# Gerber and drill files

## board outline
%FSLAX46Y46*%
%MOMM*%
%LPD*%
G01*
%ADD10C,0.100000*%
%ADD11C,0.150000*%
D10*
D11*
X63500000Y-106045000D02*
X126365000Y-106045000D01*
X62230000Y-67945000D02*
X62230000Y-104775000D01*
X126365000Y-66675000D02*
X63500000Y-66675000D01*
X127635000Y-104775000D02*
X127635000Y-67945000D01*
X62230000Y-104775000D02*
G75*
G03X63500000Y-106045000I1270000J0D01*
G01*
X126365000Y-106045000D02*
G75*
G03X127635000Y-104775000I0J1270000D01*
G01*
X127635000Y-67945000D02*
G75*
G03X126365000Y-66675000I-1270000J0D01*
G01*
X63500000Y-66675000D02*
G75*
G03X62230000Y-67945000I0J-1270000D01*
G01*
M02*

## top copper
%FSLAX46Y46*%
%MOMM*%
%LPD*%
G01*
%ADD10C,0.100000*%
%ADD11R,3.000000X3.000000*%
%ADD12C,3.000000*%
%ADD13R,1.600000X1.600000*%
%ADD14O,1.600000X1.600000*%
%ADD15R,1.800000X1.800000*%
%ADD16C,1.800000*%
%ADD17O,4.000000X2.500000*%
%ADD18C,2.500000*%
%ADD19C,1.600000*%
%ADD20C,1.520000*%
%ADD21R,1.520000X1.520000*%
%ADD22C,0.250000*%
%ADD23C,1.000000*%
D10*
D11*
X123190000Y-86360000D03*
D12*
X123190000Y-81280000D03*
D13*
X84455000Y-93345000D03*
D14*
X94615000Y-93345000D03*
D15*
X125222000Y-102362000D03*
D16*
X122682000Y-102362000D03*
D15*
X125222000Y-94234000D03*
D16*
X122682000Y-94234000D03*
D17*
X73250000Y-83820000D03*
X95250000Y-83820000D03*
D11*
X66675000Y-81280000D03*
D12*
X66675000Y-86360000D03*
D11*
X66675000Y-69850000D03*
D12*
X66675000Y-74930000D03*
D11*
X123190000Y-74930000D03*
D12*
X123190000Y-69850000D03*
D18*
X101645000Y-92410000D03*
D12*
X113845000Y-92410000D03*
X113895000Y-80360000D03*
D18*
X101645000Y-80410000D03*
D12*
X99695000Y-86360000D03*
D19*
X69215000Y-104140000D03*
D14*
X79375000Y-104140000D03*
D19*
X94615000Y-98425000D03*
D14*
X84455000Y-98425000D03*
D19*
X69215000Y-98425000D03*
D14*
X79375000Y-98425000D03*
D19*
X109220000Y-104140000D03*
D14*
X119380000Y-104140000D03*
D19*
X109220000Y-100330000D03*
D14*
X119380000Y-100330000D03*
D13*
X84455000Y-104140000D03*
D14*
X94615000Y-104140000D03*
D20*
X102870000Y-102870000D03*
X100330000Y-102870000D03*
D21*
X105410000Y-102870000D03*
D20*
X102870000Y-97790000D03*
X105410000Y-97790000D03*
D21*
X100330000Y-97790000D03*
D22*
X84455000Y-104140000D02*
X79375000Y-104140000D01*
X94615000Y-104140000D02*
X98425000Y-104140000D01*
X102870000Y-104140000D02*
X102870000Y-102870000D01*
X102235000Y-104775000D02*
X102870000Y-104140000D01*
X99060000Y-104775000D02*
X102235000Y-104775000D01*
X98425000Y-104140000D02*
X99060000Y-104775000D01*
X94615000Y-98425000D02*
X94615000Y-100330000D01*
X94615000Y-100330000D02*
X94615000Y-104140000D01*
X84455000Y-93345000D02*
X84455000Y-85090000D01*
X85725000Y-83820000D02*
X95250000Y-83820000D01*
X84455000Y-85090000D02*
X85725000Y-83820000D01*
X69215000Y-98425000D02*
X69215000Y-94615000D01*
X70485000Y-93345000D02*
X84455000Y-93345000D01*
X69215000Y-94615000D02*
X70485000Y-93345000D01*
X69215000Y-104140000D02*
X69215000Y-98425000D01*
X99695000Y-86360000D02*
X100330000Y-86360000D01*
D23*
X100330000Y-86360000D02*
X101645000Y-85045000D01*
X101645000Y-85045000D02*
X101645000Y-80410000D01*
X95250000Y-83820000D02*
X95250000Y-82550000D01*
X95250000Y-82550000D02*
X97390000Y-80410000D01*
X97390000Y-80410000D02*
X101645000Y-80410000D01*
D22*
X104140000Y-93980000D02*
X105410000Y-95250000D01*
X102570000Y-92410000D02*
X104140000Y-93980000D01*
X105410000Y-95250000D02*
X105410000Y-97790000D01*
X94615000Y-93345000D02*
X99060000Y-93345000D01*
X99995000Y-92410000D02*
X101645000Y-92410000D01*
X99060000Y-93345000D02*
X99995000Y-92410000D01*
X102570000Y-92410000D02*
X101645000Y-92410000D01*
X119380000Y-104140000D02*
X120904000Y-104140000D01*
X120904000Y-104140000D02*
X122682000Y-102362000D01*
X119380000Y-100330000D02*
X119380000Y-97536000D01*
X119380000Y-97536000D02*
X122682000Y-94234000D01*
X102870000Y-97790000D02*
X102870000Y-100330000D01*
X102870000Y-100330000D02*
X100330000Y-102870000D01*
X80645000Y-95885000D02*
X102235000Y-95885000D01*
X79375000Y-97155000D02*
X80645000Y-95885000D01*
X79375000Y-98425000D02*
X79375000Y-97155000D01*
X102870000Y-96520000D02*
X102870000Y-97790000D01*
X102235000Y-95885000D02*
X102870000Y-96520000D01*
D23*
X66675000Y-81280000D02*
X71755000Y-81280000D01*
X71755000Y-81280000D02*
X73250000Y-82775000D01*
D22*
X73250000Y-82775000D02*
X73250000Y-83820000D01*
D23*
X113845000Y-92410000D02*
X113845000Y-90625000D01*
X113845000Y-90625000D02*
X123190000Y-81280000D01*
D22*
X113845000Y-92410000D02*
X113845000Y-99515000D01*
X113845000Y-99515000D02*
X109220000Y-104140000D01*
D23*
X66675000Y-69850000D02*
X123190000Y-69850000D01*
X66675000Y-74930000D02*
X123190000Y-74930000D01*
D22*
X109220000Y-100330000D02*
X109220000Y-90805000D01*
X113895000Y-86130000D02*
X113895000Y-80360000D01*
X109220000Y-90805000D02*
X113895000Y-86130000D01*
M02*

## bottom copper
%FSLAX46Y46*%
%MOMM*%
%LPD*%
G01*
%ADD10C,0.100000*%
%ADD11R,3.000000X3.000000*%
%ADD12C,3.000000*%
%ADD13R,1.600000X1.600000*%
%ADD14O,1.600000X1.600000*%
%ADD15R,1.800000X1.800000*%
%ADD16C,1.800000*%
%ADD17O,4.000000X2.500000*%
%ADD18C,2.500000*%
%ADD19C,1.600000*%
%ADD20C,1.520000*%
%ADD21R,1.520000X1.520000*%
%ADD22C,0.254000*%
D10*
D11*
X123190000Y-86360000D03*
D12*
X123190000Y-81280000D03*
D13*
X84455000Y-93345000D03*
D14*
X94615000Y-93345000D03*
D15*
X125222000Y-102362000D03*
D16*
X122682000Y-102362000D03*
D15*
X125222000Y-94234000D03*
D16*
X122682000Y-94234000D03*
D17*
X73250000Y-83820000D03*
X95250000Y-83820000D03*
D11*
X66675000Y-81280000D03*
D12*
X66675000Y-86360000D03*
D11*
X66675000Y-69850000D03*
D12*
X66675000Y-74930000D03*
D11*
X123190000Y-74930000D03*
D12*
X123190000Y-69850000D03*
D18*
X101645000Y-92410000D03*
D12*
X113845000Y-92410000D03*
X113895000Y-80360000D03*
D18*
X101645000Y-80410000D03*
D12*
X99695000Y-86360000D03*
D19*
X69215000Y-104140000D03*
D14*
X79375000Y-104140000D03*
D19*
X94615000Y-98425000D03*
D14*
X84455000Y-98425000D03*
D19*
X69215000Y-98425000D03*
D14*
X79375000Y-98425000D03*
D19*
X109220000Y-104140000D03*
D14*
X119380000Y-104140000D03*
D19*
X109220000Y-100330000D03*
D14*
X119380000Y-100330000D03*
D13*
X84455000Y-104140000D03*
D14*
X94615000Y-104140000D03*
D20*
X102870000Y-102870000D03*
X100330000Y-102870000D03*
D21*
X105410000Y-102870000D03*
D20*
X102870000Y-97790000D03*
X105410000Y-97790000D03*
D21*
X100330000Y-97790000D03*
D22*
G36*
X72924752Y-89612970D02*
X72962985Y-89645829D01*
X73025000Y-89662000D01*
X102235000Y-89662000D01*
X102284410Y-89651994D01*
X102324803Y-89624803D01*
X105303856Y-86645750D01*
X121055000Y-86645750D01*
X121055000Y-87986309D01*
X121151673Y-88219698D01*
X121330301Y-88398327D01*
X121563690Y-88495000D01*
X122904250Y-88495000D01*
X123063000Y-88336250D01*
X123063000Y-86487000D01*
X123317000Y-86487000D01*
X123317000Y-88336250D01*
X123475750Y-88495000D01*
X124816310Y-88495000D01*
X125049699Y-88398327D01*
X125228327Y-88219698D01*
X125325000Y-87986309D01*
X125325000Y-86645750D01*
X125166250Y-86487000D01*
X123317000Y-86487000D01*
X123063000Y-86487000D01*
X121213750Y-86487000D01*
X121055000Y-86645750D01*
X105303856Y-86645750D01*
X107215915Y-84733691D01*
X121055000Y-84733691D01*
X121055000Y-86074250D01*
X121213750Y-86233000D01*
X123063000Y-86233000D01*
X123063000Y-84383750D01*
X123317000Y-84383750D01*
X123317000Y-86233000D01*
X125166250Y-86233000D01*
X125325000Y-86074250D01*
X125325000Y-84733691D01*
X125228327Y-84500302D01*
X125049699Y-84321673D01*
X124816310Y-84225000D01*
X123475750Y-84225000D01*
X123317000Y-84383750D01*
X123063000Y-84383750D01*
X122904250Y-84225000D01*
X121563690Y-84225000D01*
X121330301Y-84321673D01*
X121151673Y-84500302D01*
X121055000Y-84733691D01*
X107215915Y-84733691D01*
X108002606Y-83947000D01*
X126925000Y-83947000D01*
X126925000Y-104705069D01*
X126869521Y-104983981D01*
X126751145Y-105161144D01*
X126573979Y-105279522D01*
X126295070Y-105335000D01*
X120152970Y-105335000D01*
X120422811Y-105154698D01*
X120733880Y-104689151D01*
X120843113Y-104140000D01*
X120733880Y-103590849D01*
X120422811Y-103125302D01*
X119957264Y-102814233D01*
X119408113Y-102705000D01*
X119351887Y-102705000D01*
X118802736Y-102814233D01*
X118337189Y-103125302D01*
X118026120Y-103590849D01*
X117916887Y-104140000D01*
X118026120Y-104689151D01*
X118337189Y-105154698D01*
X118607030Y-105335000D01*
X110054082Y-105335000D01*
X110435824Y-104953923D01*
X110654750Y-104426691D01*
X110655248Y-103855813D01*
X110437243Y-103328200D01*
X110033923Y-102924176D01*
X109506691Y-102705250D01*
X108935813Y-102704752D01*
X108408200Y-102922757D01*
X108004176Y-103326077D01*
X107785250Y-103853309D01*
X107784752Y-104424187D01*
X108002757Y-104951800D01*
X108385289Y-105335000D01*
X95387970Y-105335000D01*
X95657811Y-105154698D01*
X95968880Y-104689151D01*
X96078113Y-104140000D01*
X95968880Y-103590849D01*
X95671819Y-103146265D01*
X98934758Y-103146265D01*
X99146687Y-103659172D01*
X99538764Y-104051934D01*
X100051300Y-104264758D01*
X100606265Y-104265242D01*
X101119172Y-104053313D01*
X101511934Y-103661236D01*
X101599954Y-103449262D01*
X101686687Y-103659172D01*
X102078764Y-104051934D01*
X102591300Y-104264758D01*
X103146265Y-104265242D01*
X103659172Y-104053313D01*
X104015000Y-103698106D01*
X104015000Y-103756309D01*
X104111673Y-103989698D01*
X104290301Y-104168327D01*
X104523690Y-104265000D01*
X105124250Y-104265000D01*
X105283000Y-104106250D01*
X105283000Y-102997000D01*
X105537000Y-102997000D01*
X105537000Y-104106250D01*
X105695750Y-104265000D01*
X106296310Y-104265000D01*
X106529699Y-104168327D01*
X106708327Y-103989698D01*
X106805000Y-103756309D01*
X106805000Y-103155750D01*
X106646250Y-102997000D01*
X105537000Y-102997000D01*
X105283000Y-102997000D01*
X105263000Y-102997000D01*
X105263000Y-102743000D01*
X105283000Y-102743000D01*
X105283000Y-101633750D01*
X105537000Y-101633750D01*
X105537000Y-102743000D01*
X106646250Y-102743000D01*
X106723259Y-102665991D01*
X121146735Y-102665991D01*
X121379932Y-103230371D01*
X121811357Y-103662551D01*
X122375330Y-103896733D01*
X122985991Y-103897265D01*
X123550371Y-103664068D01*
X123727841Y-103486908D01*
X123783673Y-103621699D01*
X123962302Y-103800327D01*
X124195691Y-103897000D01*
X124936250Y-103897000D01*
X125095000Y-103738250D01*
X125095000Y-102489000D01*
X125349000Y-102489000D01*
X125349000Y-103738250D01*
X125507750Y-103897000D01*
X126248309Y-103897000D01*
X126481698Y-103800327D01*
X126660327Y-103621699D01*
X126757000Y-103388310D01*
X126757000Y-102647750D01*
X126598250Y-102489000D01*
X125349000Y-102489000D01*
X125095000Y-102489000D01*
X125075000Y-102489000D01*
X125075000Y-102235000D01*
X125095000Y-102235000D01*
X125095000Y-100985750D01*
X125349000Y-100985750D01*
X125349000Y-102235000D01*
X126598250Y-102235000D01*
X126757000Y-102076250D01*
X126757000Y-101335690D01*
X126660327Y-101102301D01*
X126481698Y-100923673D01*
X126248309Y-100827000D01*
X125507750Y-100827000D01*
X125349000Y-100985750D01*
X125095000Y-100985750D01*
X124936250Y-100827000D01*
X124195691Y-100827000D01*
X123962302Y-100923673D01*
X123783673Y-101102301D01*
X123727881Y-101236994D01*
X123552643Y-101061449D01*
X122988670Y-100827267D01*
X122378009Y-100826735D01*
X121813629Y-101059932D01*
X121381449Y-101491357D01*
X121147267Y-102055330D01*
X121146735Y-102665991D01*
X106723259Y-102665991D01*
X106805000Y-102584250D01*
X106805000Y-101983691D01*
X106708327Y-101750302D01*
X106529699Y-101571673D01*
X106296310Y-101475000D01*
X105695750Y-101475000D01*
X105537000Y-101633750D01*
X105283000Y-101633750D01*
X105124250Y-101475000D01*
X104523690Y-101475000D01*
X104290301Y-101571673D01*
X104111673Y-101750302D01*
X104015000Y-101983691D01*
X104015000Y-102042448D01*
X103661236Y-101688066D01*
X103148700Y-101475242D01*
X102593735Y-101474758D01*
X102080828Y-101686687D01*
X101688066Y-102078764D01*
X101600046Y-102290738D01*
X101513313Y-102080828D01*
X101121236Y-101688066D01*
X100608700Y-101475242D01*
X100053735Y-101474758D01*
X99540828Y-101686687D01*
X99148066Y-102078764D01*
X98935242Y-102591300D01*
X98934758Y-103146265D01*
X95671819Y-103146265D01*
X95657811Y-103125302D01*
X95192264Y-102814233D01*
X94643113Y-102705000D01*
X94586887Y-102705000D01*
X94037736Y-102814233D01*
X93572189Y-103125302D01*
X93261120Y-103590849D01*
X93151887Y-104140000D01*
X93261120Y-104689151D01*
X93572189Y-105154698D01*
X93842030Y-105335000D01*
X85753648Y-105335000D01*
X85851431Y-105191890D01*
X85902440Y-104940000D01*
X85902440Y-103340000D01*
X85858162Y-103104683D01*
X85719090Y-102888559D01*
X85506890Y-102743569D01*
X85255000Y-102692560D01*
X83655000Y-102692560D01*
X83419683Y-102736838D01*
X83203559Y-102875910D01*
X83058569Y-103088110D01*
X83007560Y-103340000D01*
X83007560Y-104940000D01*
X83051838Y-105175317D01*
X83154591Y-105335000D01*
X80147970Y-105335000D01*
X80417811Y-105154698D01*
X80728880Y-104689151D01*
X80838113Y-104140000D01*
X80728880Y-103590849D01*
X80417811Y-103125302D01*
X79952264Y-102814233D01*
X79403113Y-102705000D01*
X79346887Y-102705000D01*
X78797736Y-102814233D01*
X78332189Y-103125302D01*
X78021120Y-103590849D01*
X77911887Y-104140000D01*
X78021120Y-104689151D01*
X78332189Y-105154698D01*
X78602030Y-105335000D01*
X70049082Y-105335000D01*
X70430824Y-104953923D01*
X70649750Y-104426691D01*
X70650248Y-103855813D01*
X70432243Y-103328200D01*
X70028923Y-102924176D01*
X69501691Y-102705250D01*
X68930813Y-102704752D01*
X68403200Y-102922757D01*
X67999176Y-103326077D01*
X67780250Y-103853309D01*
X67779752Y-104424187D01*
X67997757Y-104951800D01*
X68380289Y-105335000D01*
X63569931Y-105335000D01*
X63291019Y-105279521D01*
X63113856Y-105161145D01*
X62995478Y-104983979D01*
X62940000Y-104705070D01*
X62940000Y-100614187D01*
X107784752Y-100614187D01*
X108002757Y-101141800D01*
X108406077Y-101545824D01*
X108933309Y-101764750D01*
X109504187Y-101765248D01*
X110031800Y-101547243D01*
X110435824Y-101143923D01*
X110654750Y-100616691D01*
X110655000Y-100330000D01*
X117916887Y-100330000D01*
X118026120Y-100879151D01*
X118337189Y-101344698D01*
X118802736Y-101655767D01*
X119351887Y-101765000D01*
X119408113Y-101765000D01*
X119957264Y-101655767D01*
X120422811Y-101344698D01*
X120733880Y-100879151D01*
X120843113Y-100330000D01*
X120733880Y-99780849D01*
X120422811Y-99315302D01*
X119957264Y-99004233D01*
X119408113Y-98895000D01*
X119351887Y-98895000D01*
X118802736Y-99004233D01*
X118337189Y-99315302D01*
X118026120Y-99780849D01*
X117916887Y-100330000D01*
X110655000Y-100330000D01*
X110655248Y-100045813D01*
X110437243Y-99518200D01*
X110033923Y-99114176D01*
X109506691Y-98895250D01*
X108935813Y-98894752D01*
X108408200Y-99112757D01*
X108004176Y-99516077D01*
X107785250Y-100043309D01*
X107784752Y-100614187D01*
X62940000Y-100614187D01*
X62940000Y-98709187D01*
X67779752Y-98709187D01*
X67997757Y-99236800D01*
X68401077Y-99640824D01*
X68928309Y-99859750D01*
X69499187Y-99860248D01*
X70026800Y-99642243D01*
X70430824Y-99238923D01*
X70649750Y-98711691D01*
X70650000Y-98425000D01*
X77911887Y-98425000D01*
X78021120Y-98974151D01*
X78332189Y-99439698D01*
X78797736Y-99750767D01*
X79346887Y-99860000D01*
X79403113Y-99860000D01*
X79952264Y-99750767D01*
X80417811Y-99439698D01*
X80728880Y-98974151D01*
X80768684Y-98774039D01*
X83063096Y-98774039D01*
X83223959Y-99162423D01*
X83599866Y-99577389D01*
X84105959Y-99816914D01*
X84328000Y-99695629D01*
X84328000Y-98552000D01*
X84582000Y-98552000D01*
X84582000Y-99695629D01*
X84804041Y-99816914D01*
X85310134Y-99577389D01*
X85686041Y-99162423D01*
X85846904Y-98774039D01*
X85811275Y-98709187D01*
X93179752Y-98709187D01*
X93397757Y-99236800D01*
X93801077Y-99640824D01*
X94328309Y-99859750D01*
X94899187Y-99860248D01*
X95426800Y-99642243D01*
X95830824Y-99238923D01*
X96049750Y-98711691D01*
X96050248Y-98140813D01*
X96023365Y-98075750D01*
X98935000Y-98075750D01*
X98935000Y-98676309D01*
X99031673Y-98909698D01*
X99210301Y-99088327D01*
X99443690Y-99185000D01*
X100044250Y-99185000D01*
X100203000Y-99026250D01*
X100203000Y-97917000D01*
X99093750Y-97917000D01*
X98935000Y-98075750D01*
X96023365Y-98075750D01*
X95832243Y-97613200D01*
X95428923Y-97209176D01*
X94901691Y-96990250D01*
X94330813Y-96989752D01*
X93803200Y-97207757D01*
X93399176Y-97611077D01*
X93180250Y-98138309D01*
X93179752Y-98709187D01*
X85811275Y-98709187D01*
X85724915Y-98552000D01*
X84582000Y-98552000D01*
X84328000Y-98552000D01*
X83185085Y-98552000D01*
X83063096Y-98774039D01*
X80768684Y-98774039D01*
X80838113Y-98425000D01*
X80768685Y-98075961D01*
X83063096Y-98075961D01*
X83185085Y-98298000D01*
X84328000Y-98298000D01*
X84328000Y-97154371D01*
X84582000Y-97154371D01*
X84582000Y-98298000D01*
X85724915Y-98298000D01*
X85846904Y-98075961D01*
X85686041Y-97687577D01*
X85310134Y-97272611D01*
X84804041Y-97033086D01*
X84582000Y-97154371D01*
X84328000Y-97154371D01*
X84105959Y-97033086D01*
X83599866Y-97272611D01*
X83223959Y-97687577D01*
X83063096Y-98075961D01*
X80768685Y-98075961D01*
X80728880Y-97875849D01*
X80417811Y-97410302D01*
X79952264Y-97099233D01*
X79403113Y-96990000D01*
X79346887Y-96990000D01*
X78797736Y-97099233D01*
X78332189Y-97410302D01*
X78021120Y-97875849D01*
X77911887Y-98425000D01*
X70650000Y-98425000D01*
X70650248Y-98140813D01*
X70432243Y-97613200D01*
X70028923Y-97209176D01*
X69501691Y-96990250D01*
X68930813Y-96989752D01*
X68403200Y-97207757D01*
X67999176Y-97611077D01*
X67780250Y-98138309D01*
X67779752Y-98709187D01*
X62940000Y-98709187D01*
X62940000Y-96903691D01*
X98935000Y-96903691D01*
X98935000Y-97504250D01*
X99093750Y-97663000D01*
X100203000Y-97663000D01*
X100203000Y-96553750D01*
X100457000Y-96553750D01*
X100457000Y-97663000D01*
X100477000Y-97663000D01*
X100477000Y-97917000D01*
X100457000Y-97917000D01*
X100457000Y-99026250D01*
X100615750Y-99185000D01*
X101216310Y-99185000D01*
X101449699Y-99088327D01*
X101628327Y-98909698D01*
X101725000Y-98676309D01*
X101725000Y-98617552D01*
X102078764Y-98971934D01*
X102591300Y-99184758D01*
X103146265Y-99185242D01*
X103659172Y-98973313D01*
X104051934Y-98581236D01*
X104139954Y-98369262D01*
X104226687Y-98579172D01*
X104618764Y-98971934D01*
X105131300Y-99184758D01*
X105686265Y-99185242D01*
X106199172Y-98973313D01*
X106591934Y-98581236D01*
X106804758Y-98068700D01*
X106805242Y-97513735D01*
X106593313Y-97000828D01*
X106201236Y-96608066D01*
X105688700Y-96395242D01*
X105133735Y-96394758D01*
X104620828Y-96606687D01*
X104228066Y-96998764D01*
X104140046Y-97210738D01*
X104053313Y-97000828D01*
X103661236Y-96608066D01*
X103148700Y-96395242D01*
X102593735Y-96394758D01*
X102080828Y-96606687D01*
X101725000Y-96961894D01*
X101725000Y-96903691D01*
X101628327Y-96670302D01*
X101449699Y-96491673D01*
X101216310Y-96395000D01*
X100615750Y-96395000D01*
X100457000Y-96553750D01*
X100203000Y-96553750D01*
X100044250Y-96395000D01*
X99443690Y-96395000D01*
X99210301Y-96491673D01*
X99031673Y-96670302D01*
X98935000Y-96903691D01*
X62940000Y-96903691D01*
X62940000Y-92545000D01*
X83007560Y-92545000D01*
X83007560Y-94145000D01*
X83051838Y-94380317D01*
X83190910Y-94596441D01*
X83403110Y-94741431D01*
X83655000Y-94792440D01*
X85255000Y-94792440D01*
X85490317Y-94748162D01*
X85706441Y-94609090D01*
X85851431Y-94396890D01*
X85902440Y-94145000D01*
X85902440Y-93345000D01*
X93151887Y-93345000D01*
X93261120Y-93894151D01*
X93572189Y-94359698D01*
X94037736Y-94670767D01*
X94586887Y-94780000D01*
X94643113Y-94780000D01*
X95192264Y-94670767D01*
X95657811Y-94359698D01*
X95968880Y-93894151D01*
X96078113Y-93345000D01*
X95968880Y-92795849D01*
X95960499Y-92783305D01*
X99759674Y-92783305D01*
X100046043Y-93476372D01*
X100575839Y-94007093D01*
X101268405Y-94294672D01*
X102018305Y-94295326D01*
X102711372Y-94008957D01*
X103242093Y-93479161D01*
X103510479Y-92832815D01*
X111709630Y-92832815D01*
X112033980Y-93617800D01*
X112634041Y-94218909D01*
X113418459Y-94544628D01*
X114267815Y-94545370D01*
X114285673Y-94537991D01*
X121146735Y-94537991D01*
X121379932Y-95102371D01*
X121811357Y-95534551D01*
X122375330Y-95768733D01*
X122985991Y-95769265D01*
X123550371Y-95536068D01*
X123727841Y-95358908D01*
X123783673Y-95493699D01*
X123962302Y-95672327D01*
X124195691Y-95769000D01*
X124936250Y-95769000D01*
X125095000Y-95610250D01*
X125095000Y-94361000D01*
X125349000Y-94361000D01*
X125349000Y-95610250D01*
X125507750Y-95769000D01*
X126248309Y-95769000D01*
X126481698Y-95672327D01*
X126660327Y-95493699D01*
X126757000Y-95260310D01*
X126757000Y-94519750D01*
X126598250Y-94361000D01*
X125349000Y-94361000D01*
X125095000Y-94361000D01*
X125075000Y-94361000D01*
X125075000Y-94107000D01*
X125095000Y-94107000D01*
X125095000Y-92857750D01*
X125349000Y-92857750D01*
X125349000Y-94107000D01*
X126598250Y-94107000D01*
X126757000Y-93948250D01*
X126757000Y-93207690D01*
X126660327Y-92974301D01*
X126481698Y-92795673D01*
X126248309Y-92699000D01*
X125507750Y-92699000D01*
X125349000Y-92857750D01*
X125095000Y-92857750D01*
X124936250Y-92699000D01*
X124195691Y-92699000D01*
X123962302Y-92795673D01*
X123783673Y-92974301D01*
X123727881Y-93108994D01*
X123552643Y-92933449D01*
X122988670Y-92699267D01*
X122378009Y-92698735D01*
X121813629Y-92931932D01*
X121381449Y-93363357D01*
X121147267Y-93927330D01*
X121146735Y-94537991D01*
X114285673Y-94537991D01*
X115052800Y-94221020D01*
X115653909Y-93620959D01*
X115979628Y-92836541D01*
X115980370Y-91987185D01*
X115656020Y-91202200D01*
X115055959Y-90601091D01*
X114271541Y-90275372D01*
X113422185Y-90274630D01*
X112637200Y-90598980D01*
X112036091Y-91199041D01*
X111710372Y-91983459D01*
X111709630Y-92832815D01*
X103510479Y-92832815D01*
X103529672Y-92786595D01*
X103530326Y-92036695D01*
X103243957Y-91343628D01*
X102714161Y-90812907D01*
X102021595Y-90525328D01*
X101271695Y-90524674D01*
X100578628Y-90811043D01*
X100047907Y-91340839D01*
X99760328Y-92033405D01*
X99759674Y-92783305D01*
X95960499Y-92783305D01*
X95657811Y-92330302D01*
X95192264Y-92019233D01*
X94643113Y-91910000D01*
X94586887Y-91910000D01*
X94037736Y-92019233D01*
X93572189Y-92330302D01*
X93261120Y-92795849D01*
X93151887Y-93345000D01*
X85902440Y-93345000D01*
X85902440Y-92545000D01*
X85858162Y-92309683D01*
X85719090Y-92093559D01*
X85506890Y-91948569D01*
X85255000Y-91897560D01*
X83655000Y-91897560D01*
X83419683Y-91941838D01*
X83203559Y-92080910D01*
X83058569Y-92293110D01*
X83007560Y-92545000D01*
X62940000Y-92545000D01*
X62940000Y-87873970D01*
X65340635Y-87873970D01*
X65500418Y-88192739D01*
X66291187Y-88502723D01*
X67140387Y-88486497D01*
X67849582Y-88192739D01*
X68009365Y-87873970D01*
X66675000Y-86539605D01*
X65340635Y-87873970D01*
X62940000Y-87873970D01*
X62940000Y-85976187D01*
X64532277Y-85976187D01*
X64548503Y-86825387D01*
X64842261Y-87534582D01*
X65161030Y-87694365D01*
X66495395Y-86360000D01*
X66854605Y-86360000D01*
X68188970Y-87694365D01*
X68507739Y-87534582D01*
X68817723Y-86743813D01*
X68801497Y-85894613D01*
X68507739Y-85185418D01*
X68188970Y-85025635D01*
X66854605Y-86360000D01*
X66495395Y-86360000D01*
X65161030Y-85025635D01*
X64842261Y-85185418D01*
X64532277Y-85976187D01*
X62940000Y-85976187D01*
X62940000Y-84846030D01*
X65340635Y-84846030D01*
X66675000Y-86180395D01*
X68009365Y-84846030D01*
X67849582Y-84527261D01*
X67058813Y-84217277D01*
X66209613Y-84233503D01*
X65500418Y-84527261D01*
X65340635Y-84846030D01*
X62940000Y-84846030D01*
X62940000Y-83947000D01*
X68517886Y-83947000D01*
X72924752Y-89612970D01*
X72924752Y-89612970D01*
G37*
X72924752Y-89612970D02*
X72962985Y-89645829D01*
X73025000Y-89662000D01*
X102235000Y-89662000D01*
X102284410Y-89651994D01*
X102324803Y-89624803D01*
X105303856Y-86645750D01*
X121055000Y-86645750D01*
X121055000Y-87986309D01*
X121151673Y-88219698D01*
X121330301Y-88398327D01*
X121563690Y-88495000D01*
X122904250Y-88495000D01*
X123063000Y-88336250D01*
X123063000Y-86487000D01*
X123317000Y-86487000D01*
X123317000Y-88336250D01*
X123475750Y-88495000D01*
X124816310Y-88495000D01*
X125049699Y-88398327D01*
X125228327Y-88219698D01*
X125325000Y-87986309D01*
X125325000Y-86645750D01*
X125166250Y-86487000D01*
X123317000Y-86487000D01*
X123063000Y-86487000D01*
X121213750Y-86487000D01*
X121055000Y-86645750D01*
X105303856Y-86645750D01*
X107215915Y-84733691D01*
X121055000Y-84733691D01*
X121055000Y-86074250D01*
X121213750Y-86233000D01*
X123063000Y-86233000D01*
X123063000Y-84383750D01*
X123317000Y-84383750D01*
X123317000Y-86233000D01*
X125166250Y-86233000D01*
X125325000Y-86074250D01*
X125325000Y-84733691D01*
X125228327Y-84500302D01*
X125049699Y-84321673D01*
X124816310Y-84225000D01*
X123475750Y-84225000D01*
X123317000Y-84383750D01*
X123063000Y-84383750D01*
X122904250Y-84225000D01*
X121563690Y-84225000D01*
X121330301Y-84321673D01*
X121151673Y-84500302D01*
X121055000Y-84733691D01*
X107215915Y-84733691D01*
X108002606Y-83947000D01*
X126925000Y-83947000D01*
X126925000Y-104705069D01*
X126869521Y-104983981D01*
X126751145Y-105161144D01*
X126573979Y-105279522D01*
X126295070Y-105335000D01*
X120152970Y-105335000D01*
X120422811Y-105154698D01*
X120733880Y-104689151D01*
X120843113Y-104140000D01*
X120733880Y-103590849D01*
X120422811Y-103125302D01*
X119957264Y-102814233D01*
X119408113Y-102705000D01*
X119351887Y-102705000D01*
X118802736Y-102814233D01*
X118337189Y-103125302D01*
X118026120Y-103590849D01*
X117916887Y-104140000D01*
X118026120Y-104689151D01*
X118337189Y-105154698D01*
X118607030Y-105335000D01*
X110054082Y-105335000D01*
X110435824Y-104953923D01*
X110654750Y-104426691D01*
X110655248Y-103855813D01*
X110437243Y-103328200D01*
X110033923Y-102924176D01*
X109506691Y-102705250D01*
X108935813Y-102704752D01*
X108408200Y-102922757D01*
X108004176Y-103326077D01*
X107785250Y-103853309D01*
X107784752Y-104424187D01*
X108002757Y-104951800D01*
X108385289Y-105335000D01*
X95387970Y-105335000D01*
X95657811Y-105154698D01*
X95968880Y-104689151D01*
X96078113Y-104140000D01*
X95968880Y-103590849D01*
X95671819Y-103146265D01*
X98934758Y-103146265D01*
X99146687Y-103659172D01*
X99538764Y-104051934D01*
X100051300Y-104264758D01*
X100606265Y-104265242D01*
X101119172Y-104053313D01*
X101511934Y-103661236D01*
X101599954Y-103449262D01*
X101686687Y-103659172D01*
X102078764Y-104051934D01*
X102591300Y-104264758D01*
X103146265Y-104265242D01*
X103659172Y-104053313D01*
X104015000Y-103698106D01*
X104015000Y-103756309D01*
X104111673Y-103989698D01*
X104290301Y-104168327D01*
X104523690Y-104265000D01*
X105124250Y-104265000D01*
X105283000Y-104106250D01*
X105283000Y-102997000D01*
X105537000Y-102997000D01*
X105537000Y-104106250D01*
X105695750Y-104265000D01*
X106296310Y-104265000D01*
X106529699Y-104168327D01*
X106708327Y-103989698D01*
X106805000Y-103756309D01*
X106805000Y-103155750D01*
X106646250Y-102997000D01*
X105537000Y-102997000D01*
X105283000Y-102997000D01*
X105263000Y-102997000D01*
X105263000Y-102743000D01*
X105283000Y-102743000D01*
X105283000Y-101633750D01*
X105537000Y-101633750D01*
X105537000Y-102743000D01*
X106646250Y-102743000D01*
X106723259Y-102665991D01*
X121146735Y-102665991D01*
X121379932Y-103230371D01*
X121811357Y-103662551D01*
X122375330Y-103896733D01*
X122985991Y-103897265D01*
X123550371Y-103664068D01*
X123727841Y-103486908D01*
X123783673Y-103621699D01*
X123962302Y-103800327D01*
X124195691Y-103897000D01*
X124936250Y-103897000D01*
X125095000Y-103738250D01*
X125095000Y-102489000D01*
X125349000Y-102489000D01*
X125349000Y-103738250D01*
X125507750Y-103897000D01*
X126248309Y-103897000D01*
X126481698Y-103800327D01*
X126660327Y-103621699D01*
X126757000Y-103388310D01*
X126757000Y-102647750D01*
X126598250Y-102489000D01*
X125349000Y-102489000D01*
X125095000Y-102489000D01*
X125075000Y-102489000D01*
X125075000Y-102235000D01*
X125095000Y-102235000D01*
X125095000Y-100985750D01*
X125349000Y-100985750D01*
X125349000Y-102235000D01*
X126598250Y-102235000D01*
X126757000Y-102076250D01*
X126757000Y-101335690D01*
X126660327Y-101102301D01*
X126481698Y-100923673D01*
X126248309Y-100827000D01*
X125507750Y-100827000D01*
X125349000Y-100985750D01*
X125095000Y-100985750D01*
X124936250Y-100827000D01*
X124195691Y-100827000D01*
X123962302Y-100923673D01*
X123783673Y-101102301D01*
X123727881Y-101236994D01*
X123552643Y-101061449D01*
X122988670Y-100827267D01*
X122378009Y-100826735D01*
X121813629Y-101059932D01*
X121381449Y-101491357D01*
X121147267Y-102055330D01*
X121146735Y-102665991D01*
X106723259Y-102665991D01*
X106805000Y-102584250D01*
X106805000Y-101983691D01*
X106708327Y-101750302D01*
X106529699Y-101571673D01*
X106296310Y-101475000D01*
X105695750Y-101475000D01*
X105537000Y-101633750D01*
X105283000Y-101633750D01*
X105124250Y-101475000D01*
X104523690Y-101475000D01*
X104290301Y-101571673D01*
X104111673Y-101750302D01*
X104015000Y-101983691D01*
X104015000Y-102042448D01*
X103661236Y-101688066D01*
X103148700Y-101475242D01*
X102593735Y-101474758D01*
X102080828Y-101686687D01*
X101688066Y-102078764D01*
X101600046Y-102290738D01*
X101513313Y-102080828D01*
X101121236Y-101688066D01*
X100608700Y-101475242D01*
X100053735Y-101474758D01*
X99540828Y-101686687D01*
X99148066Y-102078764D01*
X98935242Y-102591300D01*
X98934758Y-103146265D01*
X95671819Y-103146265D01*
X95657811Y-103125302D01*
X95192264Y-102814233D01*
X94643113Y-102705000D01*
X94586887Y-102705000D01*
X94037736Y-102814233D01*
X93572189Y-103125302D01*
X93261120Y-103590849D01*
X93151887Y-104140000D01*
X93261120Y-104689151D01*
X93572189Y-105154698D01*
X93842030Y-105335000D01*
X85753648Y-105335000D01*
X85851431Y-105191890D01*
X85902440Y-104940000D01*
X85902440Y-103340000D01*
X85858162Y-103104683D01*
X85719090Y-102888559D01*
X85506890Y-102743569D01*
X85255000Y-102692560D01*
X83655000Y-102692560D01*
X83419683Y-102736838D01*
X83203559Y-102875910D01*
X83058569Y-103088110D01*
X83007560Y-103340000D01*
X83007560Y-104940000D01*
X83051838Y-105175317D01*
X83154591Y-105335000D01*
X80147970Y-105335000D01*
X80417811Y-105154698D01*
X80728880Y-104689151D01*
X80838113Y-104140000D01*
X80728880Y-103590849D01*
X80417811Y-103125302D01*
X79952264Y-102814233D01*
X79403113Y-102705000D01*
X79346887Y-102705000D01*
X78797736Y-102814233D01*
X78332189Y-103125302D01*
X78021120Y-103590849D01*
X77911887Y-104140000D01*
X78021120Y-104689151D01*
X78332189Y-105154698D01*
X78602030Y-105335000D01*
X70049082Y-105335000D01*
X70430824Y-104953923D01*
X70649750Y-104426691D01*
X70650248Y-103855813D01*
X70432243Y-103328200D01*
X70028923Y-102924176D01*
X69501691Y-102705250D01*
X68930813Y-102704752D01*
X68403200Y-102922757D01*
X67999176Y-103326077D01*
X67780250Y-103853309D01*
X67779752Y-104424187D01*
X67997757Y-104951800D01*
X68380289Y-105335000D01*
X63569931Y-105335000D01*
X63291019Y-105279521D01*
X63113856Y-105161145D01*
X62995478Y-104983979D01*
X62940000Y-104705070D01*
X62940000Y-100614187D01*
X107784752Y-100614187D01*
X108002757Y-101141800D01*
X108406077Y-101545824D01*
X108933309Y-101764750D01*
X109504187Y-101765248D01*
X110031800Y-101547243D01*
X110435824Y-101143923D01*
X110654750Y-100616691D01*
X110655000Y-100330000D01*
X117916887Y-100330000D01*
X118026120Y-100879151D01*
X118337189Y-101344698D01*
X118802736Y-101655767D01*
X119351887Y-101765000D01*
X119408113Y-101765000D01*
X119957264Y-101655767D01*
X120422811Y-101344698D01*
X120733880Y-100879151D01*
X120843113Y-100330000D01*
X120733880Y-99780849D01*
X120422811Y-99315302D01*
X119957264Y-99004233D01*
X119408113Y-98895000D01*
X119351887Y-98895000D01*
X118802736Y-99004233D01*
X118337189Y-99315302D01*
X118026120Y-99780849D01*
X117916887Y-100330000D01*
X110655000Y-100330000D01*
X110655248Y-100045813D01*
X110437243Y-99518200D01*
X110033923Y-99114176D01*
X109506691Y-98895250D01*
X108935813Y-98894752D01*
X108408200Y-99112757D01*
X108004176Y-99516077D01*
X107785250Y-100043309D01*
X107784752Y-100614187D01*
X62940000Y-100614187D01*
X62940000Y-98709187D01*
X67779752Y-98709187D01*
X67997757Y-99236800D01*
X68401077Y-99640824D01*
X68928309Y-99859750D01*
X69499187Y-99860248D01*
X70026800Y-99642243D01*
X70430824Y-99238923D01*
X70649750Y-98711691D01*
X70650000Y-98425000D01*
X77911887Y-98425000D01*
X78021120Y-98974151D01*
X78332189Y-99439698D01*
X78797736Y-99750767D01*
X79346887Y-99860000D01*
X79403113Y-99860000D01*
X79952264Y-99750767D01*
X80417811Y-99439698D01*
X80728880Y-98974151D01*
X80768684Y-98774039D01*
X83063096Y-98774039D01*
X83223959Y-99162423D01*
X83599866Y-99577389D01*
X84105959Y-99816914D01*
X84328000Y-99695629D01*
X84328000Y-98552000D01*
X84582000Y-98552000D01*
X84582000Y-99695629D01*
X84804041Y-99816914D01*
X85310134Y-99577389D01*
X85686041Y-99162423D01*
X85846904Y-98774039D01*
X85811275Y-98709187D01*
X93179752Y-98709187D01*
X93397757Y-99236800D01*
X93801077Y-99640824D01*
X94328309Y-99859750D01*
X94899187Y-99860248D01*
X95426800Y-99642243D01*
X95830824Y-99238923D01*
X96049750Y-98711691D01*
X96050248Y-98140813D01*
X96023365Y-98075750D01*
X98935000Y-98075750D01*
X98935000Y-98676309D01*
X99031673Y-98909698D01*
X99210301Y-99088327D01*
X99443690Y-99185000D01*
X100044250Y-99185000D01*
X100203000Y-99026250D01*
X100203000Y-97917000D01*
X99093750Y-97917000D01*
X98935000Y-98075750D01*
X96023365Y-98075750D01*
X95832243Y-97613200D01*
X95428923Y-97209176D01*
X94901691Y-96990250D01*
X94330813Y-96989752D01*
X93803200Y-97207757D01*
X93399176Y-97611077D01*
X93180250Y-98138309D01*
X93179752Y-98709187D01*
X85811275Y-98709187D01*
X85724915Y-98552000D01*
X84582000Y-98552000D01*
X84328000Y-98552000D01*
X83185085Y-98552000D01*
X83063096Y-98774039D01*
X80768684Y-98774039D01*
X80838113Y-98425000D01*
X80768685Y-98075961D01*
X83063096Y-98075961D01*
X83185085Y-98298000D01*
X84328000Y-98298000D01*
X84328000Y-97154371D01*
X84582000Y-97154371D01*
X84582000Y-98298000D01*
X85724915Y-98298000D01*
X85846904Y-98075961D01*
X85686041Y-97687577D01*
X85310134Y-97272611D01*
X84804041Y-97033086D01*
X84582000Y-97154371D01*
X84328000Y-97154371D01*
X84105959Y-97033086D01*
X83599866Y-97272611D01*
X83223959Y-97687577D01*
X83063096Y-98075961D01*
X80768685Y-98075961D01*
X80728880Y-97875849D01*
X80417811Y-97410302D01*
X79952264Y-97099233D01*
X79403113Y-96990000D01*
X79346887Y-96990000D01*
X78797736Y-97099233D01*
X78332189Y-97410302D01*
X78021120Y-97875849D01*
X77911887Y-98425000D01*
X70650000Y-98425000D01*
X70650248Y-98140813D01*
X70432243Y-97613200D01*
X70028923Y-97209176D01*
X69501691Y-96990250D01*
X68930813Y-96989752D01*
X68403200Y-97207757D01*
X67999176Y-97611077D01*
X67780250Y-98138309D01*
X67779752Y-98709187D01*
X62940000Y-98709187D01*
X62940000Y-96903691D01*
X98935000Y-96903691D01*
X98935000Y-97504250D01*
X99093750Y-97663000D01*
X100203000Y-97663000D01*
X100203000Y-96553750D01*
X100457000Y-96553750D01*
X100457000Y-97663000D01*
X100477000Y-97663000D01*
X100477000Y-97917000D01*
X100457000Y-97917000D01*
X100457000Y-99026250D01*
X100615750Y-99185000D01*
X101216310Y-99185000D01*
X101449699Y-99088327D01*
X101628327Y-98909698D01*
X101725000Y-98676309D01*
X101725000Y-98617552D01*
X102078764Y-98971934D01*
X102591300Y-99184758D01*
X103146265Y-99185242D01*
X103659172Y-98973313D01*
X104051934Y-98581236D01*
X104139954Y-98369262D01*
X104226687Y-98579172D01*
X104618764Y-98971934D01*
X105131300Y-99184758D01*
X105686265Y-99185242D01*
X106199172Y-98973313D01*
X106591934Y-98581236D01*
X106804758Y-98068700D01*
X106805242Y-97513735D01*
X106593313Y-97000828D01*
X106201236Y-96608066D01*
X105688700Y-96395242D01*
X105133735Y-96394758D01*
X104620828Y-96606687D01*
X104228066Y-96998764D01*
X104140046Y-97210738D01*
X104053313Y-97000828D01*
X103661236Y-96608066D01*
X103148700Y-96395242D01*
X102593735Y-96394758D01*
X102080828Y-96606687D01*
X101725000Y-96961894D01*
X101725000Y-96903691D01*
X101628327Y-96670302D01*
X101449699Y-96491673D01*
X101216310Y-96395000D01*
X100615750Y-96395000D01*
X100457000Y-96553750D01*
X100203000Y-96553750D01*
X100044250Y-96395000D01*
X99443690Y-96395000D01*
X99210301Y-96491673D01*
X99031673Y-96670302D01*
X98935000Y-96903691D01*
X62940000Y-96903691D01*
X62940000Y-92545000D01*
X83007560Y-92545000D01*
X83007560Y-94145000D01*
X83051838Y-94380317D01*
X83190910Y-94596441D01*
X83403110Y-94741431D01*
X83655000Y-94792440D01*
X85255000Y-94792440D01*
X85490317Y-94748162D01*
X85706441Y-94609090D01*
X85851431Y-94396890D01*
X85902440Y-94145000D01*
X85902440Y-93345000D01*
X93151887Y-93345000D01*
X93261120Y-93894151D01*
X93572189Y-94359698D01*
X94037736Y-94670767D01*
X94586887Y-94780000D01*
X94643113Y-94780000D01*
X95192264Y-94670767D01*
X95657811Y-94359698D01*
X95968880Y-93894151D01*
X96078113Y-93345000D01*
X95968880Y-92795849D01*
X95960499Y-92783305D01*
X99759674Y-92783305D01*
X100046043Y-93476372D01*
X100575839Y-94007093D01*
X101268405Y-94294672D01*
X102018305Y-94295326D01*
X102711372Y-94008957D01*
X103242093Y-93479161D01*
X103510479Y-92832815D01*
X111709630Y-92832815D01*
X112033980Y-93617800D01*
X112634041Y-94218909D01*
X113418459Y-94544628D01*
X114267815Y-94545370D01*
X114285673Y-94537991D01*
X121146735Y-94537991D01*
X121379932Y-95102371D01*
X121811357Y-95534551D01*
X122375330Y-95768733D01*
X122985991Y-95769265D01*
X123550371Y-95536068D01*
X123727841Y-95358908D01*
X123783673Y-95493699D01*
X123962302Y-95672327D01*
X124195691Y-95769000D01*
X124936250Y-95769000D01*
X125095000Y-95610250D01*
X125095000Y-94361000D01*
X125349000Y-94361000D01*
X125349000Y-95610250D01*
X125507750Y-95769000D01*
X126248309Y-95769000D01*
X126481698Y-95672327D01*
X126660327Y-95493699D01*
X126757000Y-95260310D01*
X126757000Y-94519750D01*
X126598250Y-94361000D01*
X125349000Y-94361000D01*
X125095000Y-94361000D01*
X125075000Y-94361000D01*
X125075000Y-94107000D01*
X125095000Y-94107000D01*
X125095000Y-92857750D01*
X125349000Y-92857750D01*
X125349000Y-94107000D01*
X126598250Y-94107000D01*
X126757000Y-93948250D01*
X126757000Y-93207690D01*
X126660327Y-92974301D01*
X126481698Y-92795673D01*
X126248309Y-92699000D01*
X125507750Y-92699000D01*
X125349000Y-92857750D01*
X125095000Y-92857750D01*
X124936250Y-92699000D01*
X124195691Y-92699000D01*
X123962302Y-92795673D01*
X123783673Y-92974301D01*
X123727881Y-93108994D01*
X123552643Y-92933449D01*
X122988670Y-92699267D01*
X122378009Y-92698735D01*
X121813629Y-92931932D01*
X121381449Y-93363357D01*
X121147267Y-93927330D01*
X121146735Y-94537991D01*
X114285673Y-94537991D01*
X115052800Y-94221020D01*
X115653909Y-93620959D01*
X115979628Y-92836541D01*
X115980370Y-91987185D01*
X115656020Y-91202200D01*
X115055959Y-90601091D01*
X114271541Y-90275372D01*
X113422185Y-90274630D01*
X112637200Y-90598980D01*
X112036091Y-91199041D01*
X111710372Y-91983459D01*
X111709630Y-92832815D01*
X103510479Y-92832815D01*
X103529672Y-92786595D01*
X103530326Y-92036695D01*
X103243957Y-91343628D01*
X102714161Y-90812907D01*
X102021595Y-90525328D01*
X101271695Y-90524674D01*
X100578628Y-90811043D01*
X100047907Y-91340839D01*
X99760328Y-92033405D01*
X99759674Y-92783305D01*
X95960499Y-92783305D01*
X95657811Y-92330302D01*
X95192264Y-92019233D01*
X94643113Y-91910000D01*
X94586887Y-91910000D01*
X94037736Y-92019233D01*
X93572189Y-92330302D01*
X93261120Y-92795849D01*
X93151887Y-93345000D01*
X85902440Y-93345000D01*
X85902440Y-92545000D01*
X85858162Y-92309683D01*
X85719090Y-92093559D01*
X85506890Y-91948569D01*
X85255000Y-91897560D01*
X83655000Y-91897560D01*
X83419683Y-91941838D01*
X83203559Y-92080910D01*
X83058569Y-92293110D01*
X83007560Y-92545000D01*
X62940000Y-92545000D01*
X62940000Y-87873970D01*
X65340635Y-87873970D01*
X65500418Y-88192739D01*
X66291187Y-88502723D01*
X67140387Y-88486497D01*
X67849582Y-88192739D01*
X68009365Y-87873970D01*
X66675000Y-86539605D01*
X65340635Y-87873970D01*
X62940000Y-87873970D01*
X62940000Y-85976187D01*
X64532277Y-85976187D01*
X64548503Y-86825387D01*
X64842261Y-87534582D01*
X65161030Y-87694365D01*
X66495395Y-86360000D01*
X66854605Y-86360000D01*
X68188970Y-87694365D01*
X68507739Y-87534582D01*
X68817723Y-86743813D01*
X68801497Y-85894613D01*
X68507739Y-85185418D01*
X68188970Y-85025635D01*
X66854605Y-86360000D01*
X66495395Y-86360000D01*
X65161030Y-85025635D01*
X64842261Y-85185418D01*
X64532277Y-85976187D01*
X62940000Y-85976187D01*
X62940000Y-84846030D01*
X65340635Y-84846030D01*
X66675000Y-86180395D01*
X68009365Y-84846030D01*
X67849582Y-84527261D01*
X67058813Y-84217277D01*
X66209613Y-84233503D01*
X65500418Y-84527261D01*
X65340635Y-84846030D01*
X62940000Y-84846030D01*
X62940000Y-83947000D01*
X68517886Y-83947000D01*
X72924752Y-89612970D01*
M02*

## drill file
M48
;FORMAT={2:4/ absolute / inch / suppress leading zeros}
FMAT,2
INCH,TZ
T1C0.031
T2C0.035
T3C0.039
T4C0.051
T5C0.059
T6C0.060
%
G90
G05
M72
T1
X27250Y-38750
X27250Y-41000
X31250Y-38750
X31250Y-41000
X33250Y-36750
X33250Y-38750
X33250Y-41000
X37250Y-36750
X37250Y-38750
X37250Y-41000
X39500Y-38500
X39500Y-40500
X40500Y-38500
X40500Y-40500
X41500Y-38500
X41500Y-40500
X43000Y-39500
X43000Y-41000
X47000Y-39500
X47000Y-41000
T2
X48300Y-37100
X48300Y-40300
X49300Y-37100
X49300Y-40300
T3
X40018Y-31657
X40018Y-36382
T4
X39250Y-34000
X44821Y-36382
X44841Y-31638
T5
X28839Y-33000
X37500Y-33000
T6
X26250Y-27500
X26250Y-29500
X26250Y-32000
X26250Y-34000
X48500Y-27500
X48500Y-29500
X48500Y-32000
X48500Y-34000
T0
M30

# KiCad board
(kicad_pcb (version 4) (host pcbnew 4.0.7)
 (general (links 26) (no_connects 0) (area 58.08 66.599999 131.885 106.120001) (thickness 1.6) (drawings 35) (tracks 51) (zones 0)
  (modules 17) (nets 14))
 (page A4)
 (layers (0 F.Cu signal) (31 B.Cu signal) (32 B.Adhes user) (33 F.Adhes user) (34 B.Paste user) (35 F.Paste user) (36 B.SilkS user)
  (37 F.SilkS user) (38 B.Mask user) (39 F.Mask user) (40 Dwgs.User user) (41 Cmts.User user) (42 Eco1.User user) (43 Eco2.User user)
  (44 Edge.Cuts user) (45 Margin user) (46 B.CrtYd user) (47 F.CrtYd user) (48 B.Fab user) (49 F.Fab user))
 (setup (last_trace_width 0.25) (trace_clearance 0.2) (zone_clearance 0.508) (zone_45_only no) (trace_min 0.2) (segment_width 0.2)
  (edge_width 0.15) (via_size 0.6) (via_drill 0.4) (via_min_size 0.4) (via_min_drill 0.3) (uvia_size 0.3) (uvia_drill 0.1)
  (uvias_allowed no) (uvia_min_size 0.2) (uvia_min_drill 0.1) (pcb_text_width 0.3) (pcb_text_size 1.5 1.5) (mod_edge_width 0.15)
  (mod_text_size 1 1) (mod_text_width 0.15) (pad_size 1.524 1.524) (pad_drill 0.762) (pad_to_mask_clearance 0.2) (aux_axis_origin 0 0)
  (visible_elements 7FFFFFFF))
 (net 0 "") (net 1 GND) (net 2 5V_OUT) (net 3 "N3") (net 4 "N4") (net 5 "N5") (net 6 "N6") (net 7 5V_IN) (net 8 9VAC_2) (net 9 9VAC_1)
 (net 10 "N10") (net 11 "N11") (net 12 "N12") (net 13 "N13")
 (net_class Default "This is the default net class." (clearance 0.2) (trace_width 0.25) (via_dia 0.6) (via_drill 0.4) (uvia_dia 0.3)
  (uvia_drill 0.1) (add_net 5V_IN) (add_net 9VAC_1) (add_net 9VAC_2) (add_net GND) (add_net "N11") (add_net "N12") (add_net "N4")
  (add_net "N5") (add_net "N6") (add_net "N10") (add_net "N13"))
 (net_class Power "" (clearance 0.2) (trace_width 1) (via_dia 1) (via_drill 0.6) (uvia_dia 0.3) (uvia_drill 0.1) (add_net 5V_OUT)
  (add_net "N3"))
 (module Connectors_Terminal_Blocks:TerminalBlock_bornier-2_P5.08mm (layer F.Cu) (at 123.19 86.36 90)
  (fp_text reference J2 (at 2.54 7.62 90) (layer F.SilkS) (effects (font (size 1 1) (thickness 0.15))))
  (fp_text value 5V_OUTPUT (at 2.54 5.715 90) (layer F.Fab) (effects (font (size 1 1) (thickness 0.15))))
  (pad 1 thru_hole rect (at 0 0 90) (size 3 3) (drill 1.52) (layers *.Cu *.Mask) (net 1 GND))
  (pad 2 thru_hole circle (at 5.08 0 90) (size 3 3) (drill 1.52) (layers *.Cu *.Mask) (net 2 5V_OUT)))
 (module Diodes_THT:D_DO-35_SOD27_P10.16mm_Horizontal (layer F.Cu) (at 84.455 93.345)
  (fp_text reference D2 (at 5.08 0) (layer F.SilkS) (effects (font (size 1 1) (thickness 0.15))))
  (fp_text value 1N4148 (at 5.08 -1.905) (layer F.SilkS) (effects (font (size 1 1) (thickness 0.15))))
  (pad 1 thru_hole rect (at 0 0) (size 1.6 1.6) (drill 0.8) (layers *.Cu *.Mask) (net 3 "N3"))
  (pad 2 thru_hole oval (at 10.16 0) (size 1.6 1.6) (drill 0.8) (layers *.Cu *.Mask) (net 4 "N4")))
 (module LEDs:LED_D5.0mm (layer F.Cu) (at 125.222 102.362 180)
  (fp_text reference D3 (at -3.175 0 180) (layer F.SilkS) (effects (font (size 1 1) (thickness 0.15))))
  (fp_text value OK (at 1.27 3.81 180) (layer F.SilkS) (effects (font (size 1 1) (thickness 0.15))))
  (pad 1 thru_hole rect (at 0 0 180) (size 1.8 1.8) (drill 0.9) (layers *.Cu *.Mask) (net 1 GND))
  (pad 2 thru_hole circle (at 2.54 0 180) (size 1.8 1.8) (drill 0.9) (layers *.Cu *.Mask) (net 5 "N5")))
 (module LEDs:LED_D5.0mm (layer F.Cu) (at 125.222 94.234 180)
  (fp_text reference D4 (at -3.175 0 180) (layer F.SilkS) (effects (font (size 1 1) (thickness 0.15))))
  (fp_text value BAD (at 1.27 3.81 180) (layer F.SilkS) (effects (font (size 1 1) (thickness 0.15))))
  (pad 1 thru_hole rect (at 0 0 180) (size 1.8 1.8) (drill 0.9) (layers *.Cu *.Mask) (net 1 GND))
  (pad 2 thru_hole circle (at 2.54 0 180) (size 1.8 1.8) (drill 0.9) (layers *.Cu *.Mask) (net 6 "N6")))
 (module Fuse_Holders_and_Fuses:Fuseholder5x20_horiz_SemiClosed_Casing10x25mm (layer F.Cu) (at 95.25 83.82 180)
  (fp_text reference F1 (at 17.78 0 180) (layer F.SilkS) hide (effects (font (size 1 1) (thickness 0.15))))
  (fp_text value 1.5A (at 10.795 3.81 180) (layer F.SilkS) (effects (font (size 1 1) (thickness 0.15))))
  (pad 2 thru_hole oval (at 22 0 90) (size 2.5 4) (drill 1.5) (layers *.Cu *.Mask) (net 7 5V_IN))
  (pad 1 thru_hole oval (at 0 0 90) (size 2.5 4) (drill 1.5) (layers *.Cu *.Mask) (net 3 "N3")))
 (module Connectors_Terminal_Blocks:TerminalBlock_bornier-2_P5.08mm (layer F.Cu) (at 66.675 81.28 270)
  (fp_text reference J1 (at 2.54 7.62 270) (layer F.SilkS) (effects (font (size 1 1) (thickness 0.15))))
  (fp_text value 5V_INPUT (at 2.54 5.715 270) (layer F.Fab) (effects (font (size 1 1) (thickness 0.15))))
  (pad 1 thru_hole rect (at 0 0 270) (size 3 3) (drill 1.52) (layers *.Cu *.Mask) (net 7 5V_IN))
  (pad 2 thru_hole circle (at 5.08 0 270) (size 3 3) (drill 1.52) (layers *.Cu *.Mask) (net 1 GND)))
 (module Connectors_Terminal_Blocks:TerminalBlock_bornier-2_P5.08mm (layer F.Cu) (at 66.675 69.85 270)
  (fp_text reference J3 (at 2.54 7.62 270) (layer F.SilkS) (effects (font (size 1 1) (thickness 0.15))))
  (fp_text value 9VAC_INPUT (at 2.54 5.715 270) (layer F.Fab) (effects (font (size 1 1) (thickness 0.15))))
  (pad 1 thru_hole rect (at 0 0 270) (size 3 3) (drill 1.52) (layers *.Cu *.Mask) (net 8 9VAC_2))
  (pad 2 thru_hole circle (at 5.08 0 270) (size 3 3) (drill 1.52) (layers *.Cu *.Mask) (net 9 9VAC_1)))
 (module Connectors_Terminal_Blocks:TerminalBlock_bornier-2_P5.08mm (layer F.Cu) (at 123.19 74.93 90)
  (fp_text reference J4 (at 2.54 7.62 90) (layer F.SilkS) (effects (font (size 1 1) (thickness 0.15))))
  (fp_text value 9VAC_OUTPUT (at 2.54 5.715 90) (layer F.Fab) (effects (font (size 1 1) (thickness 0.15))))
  (pad 1 thru_hole rect (at 0 0 90) (size 3 3) (drill 1.52) (layers *.Cu *.Mask) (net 9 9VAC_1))
  (pad 2 thru_hole circle (at 5.08 0 90) (size 3 3) (drill 1.52) (layers *.Cu *.Mask) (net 8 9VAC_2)))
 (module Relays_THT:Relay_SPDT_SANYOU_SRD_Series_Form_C (layer F.Cu) (at 99.695 86.36)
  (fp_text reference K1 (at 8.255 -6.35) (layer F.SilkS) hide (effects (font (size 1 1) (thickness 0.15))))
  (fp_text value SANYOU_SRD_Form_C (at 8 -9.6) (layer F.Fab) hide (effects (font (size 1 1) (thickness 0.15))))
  (pad 2 thru_hole circle (at 1.95 6.05 90) (size 2.5 2.5) (drill 1) (layers *.Cu *.Mask) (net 4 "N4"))
  (pad 3 thru_hole circle (at 14.15 6.05 90) (size 3 3) (drill 1.3) (layers *.Cu *.Mask) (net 2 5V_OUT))
  (pad 4 thru_hole circle (at 14.2 -6 90) (size 3 3) (drill 1.3) (layers *.Cu *.Mask) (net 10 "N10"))
  (pad 5 thru_hole circle (at 1.95 -5.95 90) (size 2.5 2.5) (drill 1) (layers *.Cu *.Mask) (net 3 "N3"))
  (pad 1 thru_hole circle (at 0 0 90) (size 3 3) (drill 1.3) (layers *.Cu *.Mask) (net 3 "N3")))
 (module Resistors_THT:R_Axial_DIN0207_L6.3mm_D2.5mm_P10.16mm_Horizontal (layer F.Cu) (at 69.215 104.14)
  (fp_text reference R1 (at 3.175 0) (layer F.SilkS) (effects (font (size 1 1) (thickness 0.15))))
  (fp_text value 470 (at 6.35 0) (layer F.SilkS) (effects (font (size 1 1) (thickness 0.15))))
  (pad 1 thru_hole circle (at 0 0) (size 1.6 1.6) (drill 0.8) (layers *.Cu *.Mask) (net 3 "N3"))
  (pad 2 thru_hole oval (at 10.16 0) (size 1.6 1.6) (drill 0.8) (layers *.Cu *.Mask) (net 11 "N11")))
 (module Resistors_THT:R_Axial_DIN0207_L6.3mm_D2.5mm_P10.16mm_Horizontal (layer F.Cu) (at 94.615 98.425 180)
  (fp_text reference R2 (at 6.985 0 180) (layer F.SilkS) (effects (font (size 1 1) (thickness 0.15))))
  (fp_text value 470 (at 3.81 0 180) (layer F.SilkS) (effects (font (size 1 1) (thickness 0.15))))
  (pad 1 thru_hole circle (at 0 0 180) (size 1.6 1.6) (drill 0.8) (layers *.Cu *.Mask) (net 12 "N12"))
  (pad 2 thru_hole oval (at 10.16 0 180) (size 1.6 1.6) (drill 0.8) (layers *.Cu *.Mask) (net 1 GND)))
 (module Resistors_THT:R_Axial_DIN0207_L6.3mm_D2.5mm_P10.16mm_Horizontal (layer F.Cu) (at 69.215 98.425)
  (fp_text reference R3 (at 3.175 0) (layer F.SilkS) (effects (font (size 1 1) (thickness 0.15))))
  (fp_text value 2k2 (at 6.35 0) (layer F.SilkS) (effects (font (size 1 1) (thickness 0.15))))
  (pad 1 thru_hole circle (at 0 0) (size 1.6 1.6) (drill 0.8) (layers *.Cu *.Mask) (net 3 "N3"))
  (pad 2 thru_hole oval (at 10.16 0) (size 1.6 1.6) (drill 0.8) (layers *.Cu *.Mask) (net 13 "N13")))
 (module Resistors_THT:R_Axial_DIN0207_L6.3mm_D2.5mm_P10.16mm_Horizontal (layer F.Cu) (at 109.22 104.14)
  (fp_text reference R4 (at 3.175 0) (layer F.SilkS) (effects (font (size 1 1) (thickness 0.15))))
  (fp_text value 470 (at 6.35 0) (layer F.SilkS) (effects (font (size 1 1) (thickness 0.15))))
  (pad 1 thru_hole circle (at 0 0) (size 1.6 1.6) (drill 0.8) (layers *.Cu *.Mask) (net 2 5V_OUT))
  (pad 2 thru_hole oval (at 10.16 0) (size 1.6 1.6) (drill 0.8) (layers *.Cu *.Mask) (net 5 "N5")))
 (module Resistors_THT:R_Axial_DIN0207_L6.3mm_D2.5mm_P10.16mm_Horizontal (layer F.Cu) (at 109.22 100.33)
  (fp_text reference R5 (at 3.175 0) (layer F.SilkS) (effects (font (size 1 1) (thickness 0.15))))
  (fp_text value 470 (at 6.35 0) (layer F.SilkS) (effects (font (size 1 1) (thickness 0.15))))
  (pad 1 thru_hole circle (at 0 0) (size 1.6 1.6) (drill 0.8) (layers *.Cu *.Mask) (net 10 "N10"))
  (pad 2 thru_hole oval (at 10.16 0) (size 1.6 1.6) (drill 0.8) (layers *.Cu *.Mask) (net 6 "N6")))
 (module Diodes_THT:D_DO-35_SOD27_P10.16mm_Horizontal (layer F.Cu) (at 84.455 104.14)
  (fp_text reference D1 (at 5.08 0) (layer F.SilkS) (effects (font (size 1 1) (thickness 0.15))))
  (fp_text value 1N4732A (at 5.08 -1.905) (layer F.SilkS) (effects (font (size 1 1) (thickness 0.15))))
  (pad 1 thru_hole rect (at 0 0) (size 1.6 1.6) (drill 0.8) (layers *.Cu *.Mask) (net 11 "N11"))
  (pad 2 thru_hole oval (at 10.16 0) (size 1.6 1.6) (drill 0.8) (layers *.Cu *.Mask) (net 12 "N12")))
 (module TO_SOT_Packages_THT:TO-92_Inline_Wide (layer F.Cu) (at 105.41 102.87 180)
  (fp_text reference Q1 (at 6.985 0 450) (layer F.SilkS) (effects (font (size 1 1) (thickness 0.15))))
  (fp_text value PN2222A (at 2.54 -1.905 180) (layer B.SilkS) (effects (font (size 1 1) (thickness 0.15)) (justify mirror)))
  (pad 2 thru_hole circle (at 2.54 0 270) (size 1.52 1.52) (drill 0.8) (layers *.Cu *.Mask) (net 12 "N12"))
  (pad 3 thru_hole circle (at 5.08 0 270) (size 1.52 1.52) (drill 0.8) (layers *.Cu *.Mask) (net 13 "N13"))
  (pad 1 thru_hole rect (at 0 0 270) (size 1.52 1.52) (drill 0.8) (layers *.Cu *.Mask) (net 1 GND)))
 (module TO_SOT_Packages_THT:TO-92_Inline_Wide (layer F.Cu) (at 100.33 97.79)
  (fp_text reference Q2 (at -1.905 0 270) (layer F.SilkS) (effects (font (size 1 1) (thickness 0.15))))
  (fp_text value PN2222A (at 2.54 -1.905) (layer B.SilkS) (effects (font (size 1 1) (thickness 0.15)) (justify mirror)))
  (pad 2 thru_hole circle (at 2.54 0 90) (size 1.52 1.52) (drill 0.8) (layers *.Cu *.Mask) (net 13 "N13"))
  (pad 3 thru_hole circle (at 5.08 0 90) (size 1.52 1.52) (drill 0.8) (layers *.Cu *.Mask) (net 4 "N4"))
  (pad 1 thru_hole rect (at 0 0 90) (size 1.52 1.52) (drill 0.8) (layers *.Cu *.Mask) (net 1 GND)))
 (gr_line (start 63.5 106.045) (end 126.365 106.045) (angle 90) (layer Edge.Cuts) (width 0.15))
 (gr_line (start 62.23 67.945) (end 62.23 104.775) (angle 90) (layer Edge.Cuts) (width 0.15))
 (gr_line (start 126.365 66.675) (end 63.5 66.675) (angle 90) (layer Edge.Cuts) (width 0.15))
 (gr_line (start 127.635 104.775) (end 127.635 67.945) (angle 90) (layer Edge.Cuts) (width 0.15))
 (gr_arc (start 63.5 104.775) (end 63.5 106.045) (angle 90) (layer Edge.Cuts) (width 0.15))
 (gr_arc (start 126.365 104.775) (end 127.635 104.775) (angle 90) (layer Edge.Cuts) (width 0.15))
 (gr_arc (start 126.365 67.945) (end 126.365 66.675) (angle 90) (layer Edge.Cuts) (width 0.15))
 (gr_arc (start 63.5 67.945) (end 62.23 67.945) (angle 90) (layer Edge.Cuts) (width 0.15))
 (segment (start 84.455 104.14) (end 79.375 104.14) (width 0.25) (layer F.Cu) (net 11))
 (segment (start 94.615 104.14) (end 98.425 104.14) (width 0.25) (layer F.Cu) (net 12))
 (segment (start 102.87 104.14) (end 102.87 102.87) (width 0.25) (layer F.Cu) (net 12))
 (segment (start 102.235 104.775) (end 102.87 104.14) (width 0.25) (layer F.Cu) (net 12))
 (segment (start 99.06 104.775) (end 102.235 104.775) (width 0.25) (layer F.Cu) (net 12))
 (segment (start 98.425 104.14) (end 99.06 104.775) (width 0.25) (layer F.Cu) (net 12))
 (segment (start 94.615 98.425) (end 94.615 100.33) (width 0.25) (layer F.Cu) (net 12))
 (segment (start 94.615 100.33) (end 94.615 104.14) (width 0.25) (layer F.Cu) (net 12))
 (segment (start 84.455 93.345) (end 84.455 85.09) (width 0.25) (layer F.Cu) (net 3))
 (segment (start 85.725 83.82) (end 95.25 83.82) (width 0.25) (layer F.Cu) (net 3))
 (segment (start 84.455 85.09) (end 85.725 83.82) (width 0.25) (layer F.Cu) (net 3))
 (segment (start 69.215 98.425) (end 69.215 94.615) (width 0.25) (layer F.Cu) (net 3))
 (segment (start 70.485 93.345) (end 84.455 93.345) (width 0.25) (layer F.Cu) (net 3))
 (segment (start 69.215 94.615) (end 70.485 93.345) (width 0.25) (layer F.Cu) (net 3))
 (segment (start 69.215 104.14) (end 69.215 98.425) (width 0.25) (layer F.Cu) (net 3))
 (segment (start 99.695 86.36) (end 100.33 86.36) (width 0.25) (layer F.Cu) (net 3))
 (segment (start 100.33 86.36) (end 101.645 85.045) (width 1) (layer F.Cu) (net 3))
 (segment (start 101.645 85.045) (end 101.645 80.41) (width 1) (layer F.Cu) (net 3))
 (segment (start 95.25 83.82) (end 95.25 82.55) (width 1) (layer F.Cu) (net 3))
 (segment (start 95.25 82.55) (end 97.39 80.41) (width 1) (layer F.Cu) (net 3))
 (segment (start 97.39 80.41) (end 101.645 80.41) (width 1) (layer F.Cu) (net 3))
 (segment (start 104.14 93.98) (end 105.41 95.25) (width 0.25) (layer F.Cu) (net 4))
 (segment (start 102.57 92.41) (end 104.14 93.98) (width 0.25) (layer F.Cu) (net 4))
 (segment (start 105.41 95.25) (end 105.41 97.79) (width 0.25) (layer F.Cu) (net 4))
 (segment (start 94.615 93.345) (end 99.06 93.345) (width 0.25) (layer F.Cu) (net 4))
 (segment (start 99.995 92.41) (end 101.645 92.41) (width 0.25) (layer F.Cu) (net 4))
 (segment (start 99.06 93.345) (end 99.995 92.41) (width 0.25) (layer F.Cu) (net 4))
 (segment (start 102.57 92.41) (end 101.645 92.41) (width 0.25) (layer F.Cu) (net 4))
 (segment (start 119.38 104.14) (end 120.904 104.14) (width 0.25) (layer F.Cu) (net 5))
 (segment (start 120.904 104.14) (end 122.682 102.362) (width 0.25) (layer F.Cu) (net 5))
 (segment (start 119.38 100.33) (end 119.38 97.536) (width 0.25) (layer F.Cu) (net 6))
 (segment (start 119.38 97.536) (end 122.682 94.234) (width 0.25) (layer F.Cu) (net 6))
 (segment (start 102.87 97.79) (end 102.87 100.33) (width 0.25) (layer F.Cu) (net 13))
 (segment (start 102.87 100.33) (end 100.33 102.87) (width 0.25) (layer F.Cu) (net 13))
 (segment (start 80.645 95.885) (end 102.235 95.885) (width 0.25) (layer F.Cu) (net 13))
 (segment (start 79.375 97.155) (end 80.645 95.885) (width 0.25) (layer F.Cu) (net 13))
 (segment (start 79.375 98.425) (end 79.375 97.155) (width 0.25) (layer F.Cu) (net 13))
 (segment (start 102.87 96.52) (end 102.87 97.79) (width 0.25) (layer F.Cu) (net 13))
 (segment (start 102.235 95.885) (end 102.87 96.52) (width 0.25) (layer F.Cu) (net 13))
 (segment (start 66.675 81.28) (end 71.755 81.28) (width 1) (layer F.Cu) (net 7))
 (segment (start 71.755 81.28) (end 73.25 82.775) (width 1) (layer F.Cu) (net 7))
 (segment (start 73.25 82.775) (end 73.25 83.82) (width 0.25) (layer F.Cu) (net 7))
 (segment (start 113.845 92.41) (end 113.845 90.625) (width 1) (layer F.Cu) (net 2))
 (segment (start 113.845 90.625) (end 123.19 81.28) (width 1) (layer F.Cu) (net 2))
 (segment (start 113.845 92.41) (end 113.845 99.515) (width 0.25) (layer F.Cu) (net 2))
 (segment (start 113.845 99.515) (end 109.22 104.14) (width 0.25) (layer F.Cu) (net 2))
 (segment (start 66.675 69.85) (end 123.19 69.85) (width 1) (layer F.Cu) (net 8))
 (segment (start 66.675 74.93) (end 123.19 74.93) (width 1) (layer F.Cu) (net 9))
 (segment (start 109.22 100.33) (end 109.22 90.805) (width 0.25) (layer F.Cu) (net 10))
 (segment (start 113.895 86.13) (end 113.895 80.36) (width 0.25) (layer F.Cu) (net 10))
 (segment (start 109.22 90.805) (end 113.895 86.13) (width 0.25) (layer F.Cu) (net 10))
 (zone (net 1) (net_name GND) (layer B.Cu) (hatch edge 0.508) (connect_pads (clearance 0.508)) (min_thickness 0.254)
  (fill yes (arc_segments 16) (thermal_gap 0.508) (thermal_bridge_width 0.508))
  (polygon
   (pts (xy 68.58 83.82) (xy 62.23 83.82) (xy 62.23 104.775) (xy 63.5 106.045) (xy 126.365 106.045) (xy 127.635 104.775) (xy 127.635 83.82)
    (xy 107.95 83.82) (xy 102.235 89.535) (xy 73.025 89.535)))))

